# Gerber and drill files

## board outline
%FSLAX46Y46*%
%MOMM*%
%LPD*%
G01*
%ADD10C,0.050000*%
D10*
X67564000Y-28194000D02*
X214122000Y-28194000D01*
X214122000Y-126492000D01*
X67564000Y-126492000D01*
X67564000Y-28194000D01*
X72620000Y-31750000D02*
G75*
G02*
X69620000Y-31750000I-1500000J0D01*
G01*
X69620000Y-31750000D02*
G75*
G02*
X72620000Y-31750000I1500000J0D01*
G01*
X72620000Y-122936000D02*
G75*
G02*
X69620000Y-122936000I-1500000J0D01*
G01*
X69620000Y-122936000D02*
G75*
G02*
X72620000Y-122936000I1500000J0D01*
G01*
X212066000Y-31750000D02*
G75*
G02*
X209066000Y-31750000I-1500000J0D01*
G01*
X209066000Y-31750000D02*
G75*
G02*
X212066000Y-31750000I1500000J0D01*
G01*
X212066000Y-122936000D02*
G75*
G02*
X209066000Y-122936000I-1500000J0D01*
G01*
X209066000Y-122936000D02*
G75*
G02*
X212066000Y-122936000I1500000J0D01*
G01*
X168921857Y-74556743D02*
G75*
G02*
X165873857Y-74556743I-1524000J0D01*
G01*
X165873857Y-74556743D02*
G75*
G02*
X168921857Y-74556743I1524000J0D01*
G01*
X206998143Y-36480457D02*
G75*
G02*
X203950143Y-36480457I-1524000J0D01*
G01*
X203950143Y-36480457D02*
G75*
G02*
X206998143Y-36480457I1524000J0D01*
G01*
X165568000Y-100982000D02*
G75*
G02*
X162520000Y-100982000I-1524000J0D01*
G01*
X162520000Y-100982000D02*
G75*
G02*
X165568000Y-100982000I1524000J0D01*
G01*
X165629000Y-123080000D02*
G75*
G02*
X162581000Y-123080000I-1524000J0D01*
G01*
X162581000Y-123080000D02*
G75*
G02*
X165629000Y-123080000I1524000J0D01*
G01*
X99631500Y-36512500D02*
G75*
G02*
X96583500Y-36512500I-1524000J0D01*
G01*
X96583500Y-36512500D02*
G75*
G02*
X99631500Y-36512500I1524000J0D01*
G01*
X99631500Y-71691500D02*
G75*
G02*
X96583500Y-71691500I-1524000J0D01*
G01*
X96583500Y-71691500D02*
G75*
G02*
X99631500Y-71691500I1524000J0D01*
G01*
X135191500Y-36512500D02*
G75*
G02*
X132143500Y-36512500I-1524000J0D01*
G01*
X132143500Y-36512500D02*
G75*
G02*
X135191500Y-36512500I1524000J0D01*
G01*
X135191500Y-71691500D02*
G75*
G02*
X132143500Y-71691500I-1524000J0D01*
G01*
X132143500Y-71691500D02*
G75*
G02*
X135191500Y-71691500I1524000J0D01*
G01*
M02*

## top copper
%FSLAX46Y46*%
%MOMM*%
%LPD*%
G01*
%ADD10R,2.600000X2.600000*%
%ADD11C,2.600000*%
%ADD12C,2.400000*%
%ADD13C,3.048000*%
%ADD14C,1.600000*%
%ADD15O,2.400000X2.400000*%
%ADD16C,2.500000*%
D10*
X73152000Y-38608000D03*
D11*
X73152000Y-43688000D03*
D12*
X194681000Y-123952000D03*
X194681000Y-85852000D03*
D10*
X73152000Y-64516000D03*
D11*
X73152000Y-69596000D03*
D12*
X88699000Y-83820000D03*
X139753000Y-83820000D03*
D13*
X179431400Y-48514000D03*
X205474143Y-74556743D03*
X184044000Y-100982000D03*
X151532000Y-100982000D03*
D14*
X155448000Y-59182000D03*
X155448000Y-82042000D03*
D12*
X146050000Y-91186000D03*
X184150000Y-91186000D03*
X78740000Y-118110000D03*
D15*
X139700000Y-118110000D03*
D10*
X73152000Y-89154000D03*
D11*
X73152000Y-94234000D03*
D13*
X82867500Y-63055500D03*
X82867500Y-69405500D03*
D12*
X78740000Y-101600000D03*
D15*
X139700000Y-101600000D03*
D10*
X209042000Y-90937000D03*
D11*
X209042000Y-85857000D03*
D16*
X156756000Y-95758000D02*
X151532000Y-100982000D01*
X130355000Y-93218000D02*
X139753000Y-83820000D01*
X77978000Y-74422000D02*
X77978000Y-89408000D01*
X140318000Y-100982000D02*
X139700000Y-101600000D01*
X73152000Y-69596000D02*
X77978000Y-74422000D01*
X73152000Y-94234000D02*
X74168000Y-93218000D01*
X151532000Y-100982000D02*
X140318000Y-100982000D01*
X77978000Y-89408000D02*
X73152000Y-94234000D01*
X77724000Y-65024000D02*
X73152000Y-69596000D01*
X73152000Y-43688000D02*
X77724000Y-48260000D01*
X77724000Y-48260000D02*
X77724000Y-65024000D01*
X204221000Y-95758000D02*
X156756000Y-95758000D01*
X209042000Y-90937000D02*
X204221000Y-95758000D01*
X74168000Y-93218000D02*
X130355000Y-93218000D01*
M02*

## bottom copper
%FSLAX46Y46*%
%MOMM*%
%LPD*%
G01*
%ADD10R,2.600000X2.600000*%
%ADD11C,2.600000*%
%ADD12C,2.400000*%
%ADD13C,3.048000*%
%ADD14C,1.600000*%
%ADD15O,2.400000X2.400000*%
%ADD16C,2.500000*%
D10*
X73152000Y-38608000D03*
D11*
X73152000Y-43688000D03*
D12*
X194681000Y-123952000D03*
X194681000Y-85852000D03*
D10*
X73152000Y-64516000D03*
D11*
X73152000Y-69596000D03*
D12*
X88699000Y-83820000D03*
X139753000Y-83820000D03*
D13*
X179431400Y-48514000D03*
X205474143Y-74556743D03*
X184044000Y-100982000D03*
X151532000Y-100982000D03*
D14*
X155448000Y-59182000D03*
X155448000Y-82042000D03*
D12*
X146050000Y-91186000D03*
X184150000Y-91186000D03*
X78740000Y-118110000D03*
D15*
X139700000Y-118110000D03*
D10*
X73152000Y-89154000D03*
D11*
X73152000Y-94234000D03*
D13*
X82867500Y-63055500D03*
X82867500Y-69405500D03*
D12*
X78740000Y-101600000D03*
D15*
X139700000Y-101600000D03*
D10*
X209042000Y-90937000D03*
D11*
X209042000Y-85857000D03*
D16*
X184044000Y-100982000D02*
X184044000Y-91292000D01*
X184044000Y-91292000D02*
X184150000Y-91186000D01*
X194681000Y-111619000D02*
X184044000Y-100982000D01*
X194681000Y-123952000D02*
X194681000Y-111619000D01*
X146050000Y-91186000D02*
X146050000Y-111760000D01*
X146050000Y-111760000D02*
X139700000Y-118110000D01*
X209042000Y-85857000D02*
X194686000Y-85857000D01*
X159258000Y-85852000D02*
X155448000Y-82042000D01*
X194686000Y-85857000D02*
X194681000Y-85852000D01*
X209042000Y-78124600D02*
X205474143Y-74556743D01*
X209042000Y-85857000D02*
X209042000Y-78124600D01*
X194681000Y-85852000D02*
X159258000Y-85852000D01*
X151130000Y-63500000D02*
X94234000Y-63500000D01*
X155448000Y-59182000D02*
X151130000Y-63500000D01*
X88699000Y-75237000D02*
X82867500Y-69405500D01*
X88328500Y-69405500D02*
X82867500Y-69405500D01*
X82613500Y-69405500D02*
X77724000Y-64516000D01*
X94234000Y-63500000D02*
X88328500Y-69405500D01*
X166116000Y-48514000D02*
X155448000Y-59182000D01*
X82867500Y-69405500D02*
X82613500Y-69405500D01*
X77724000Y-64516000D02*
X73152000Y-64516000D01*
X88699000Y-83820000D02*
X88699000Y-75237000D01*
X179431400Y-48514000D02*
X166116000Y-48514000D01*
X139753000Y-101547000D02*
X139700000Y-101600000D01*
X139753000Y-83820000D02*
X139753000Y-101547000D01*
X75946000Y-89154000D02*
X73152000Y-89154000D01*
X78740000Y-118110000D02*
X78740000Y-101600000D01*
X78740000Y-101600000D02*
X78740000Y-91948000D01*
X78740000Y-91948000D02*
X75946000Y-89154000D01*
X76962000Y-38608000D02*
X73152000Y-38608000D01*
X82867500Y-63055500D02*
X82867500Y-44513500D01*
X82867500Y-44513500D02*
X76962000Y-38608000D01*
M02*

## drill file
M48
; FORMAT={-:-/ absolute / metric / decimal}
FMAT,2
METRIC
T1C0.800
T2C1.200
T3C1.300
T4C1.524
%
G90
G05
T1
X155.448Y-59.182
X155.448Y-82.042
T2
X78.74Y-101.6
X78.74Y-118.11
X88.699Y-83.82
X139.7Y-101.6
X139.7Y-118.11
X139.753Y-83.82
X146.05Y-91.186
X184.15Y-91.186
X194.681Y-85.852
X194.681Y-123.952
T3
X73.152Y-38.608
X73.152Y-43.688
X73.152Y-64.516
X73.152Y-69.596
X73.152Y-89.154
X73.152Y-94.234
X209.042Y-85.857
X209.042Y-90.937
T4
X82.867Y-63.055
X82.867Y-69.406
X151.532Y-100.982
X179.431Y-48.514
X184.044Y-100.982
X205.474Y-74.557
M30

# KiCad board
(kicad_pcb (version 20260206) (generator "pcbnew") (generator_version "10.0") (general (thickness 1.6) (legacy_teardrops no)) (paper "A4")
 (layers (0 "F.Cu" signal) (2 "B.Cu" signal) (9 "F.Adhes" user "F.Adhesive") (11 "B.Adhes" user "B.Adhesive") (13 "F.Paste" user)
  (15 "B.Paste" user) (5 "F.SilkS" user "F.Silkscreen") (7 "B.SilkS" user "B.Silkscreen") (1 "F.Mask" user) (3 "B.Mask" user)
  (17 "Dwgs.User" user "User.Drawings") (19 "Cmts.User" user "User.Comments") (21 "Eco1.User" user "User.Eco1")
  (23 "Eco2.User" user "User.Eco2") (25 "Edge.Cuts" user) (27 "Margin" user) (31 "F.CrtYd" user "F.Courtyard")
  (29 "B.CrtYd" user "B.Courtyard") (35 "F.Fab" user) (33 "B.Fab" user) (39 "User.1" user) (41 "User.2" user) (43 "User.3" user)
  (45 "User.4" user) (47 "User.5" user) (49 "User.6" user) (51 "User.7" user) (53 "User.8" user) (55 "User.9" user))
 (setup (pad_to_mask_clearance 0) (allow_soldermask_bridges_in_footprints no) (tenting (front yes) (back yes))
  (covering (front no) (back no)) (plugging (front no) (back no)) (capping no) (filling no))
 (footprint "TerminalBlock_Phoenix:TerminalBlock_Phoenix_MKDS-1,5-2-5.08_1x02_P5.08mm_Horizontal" (layer "F.Cu") (at 73.152 38.608 -90)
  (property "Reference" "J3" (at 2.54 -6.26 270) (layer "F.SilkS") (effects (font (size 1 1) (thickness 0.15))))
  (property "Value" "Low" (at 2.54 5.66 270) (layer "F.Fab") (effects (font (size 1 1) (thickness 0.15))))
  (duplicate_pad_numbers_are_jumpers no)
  (pad "1" thru_hole rect (at 0 0 270) (size 2.6 2.6) (drill 1.3) (layers "*.Cu" "*.Mask") (remove_unused_layers no) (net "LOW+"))
  (pad "2" thru_hole circle (at 5.08 0 270) (size 2.6 2.6) (drill 1.3) (layers "*.Cu" "*.Mask") (remove_unused_layers no) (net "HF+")))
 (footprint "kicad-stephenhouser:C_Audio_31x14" (layer "F.Cu") (at 194.681 123.952 90)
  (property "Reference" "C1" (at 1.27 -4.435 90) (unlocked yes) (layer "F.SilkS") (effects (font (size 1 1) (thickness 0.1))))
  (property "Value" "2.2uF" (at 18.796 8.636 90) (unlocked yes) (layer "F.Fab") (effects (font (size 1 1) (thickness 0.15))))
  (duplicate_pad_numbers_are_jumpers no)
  (pad "1" thru_hole circle (at 0 0 90) (size 2.4 2.4) (drill 1.2) (layers "*.Cu" "*.Mask") (remove_unused_layers no) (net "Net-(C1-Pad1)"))
  (pad "2" thru_hole circle (at 38.1 0 90) (size 2.4 2.4) (drill 1.2) (layers "*.Cu" "*.Mask") (remove_unused_layers no) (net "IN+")))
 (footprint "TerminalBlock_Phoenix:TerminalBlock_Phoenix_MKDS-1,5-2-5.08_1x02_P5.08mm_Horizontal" (layer "F.Cu") (at 73.152 64.516 -90)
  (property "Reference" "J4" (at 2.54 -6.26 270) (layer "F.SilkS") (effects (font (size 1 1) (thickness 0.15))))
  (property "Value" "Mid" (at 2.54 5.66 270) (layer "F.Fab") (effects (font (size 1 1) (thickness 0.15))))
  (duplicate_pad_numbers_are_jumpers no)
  (pad "1" thru_hole rect (at 0 0 270) (size 2.6 2.6) (drill 1.3) (layers "*.Cu" "*.Mask") (remove_unused_layers no) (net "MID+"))
  (pad "2" thru_hole circle (at 5.08 0 270) (size 2.6 2.6) (drill 1.3) (layers "*.Cu" "*.Mask") (remove_unused_layers no) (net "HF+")))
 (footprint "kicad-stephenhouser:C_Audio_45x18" (layer "F.Cu") (at 88.699 83.82)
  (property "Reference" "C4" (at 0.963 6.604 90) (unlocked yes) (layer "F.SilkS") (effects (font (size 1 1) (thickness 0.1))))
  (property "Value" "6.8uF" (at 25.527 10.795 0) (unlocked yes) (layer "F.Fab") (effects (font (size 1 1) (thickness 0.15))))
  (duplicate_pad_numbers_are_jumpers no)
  (pad "1" thru_hole circle (at 0 0) (size 2.4 2.4) (drill 1.2) (layers "*.Cu" "*.Mask") (remove_unused_layers no) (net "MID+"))
  (pad "2" thru_hole circle (at 51.054 0) (size 2.4 2.4) (drill 1.2) (layers "*.Cu" "*.Mask") (remove_unused_layers no) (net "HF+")))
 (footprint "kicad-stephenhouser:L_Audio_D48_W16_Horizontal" (layer "F.Cu") (at 186.436 55.5186 -45)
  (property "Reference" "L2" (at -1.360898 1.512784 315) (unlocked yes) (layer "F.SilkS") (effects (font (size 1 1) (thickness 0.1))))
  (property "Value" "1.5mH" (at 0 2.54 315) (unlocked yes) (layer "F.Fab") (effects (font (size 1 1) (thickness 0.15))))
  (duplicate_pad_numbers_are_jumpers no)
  (fp_circle (center 0 26.924) (end 1.524 26.924) (stroke (width 0.05) (type default)) (fill no) (layer "Edge.Cuts"))
  (fp_circle (center 0 -26.924) (end 1.524 -26.924) (stroke (width 0.05) (type default)) (fill no) (layer "Edge.Cuts"))
  (pad "1" thru_hole circle (at -9.906 0 315) (size 3.048 3.048) (drill 1.524) (layers "*.Cu" "*.Mask") (remove_unused_layers no)
   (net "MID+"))
  (pad "2" thru_hole circle (at 26.924 0 315) (size 3.048 3.048) (drill 1.524) (layers "*.Cu" "*.Mask") (remove_unused_layers no)
   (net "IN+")))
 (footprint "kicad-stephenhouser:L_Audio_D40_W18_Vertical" (layer "F.Cu") (at 184.044 100.982 180)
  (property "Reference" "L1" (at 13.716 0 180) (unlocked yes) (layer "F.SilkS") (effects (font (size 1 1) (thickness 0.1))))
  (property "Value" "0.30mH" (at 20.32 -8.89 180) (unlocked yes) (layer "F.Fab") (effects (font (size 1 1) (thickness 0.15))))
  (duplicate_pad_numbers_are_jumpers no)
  (fp_circle (center 20 0) (end 21.524 0) (stroke (width 0.05) (type default)) (fill no) (layer "Edge.Cuts"))
  (fp_circle (center 19.939 -22.098) (end 21.463 -22.098) (stroke (width 0.05) (type default)) (fill no) (layer "Edge.Cuts"))
  (pad "1" thru_hole circle (at 0 0 180) (size 3.048 3.048) (drill 1.524) (layers "*.Cu" "*.Mask") (remove_unused_layers no)
   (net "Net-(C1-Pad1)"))
  (pad "2" thru_hole circle (at 32.512 0 180) (size 3.048 3.048) (drill 1.524) (layers "*.Cu" "*.Mask") (remove_unused_layers no)
   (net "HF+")))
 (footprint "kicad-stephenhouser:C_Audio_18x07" (layer "F.Cu") (at 155.448 59.182 -90)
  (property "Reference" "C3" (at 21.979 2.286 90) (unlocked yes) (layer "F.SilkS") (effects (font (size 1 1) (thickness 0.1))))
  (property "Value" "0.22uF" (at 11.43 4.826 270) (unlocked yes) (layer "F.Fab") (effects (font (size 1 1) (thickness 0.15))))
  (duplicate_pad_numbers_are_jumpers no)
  (pad "1" thru_hole circle (at 0 0 270) (size 1.6 1.6) (drill 0.8) (layers "*.Cu" "*.Mask") (remove_unused_layers no) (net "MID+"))
  (pad "2" thru_hole circle (at 22.86 0 270) (size 1.6 1.6) (drill 0.8) (layers "*.Cu" "*.Mask") (remove_unused_layers no) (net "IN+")))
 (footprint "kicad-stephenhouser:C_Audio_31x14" (layer "F.Cu") (at 146.05 91.186)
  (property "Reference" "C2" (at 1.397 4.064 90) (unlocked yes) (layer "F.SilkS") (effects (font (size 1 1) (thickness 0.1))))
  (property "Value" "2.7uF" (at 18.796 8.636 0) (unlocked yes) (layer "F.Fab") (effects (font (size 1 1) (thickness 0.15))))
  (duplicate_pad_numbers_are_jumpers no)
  (pad "1" thru_hole circle (at 0 0) (size 2.4 2.4) (drill 1.2) (layers "*.Cu" "*.Mask") (remove_unused_layers no) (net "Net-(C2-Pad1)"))
  (pad "2" thru_hole circle (at 38.1 0) (size 2.4 2.4) (drill 1.2) (layers "*.Cu" "*.Mask") (remove_unused_layers no) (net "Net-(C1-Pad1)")))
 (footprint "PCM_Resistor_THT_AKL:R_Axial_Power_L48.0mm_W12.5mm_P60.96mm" (layer "F.Cu") (at 78.74 118.11)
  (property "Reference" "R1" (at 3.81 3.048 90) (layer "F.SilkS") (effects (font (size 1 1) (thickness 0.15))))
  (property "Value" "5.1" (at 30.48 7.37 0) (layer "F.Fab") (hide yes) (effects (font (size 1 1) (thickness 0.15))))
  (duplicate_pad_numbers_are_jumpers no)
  (pad "1" thru_hole circle (at 0 0) (size 2.4 2.4) (drill 1.2) (layers "*.Cu" "*.Mask") (remove_unused_layers no) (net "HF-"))
  (pad "2" thru_hole oval (at 60.96 0) (size 2.4 2.4) (drill 1.2) (layers "*.Cu" "*.Mask") (remove_unused_layers no) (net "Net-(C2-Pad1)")))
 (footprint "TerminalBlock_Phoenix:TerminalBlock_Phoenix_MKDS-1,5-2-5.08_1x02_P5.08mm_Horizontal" (layer "F.Cu") (at 73.152 89.154 -90)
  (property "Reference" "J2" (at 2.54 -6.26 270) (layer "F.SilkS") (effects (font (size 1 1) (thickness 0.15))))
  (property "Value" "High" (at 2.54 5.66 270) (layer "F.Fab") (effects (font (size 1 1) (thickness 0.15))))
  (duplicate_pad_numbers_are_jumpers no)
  (pad "1" thru_hole rect (at 0 0 270) (size 2.6 2.6) (drill 1.3) (layers "*.Cu" "*.Mask") (remove_unused_layers no) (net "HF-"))
  (pad "2" thru_hole circle (at 5.08 0 270) (size 2.6 2.6) (drill 1.3) (layers "*.Cu" "*.Mask") (remove_unused_layers no) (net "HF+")))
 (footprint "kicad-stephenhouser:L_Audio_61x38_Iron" (layer "F.Cu") (at 82.8675 69.4055)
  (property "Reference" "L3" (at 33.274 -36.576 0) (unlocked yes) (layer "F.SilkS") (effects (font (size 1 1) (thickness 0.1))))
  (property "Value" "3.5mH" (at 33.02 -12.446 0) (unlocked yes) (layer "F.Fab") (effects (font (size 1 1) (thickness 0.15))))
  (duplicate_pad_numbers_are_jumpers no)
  (fp_circle (center 15.24 -32.893) (end 16.764 -32.893) (stroke (width 0.05) (type default)) (fill no) (layer "Edge.Cuts"))
  (fp_circle (center 15.24 2.286) (end 16.764 2.286) (stroke (width 0.05) (type default)) (fill no) (layer "Edge.Cuts"))
  (fp_circle (center 50.8 -32.893) (end 52.324 -32.893) (stroke (width 0.05) (type default)) (fill no) (layer "Edge.Cuts"))
  (fp_circle (center 50.8 2.286) (end 52.324 2.286) (stroke (width 0.05) (type default)) (fill no) (layer "Edge.Cuts"))
  (pad "1" thru_hole circle (at 0 -6.35) (size 3.048 3.048) (drill 1.524) (layers "*.Cu" "*.Mask") (remove_unused_layers no) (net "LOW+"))
  (pad "2" thru_hole circle (at 0 0) (size 3.048 3.048) (drill 1.524) (layers "*.Cu" "*.Mask") (remove_unused_layers no) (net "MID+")))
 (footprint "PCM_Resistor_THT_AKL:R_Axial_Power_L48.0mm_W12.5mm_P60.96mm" (layer "F.Cu") (at 78.74 101.6)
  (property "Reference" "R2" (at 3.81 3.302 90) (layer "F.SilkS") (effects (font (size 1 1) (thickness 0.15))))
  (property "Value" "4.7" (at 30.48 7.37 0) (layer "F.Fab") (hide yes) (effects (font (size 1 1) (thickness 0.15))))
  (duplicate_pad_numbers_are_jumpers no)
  (pad "1" thru_hole circle (at 0 0) (size 2.4 2.4) (drill 1.2) (layers "*.Cu" "*.Mask") (remove_unused_layers no) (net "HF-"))
  (pad "2" thru_hole oval (at 60.96 0) (size 2.4 2.4) (drill 1.2) (layers "*.Cu" "*.Mask") (remove_unused_layers no) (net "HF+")))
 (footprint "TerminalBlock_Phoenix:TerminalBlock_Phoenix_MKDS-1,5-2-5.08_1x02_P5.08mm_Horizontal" (layer "F.Cu") (at 209.042 90.937 90)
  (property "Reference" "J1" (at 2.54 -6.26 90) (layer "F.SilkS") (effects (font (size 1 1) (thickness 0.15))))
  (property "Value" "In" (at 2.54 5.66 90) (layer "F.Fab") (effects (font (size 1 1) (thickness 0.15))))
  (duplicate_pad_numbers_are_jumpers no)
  (pad "1" thru_hole rect (at 0 0 90) (size 2.6 2.6) (drill 1.3) (layers "*.Cu" "*.Mask") (remove_unused_layers no) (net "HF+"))
  (pad "2" thru_hole circle (at 5.08 0 90) (size 2.6 2.6) (drill 1.3) (layers "*.Cu" "*.Mask") (remove_unused_layers no) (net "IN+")))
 (gr_rect (start 67.564 28.194) (end 214.122 126.492) (stroke (width 0.05) (type default)) (fill no) (layer "Edge.Cuts"))
 (gr_circle (center 71.12 31.75) (end 72.62 31.75) (stroke (width 0.05) (type default)) (fill no) (layer "Edge.Cuts"))
 (gr_circle (center 71.12 122.936) (end 72.62 122.936) (stroke (width 0.05) (type default)) (fill no) (layer "Edge.Cuts"))
 (gr_circle (center 210.566 31.75) (end 212.066 31.75) (stroke (width 0.05) (type default)) (fill no) (layer "Edge.Cuts"))
 (gr_circle (center 210.566 122.936) (end 212.066 122.936) (stroke (width 0.05) (type default)) (fill no) (layer "Edge.Cuts"))
 (segment (start 184.044 100.982) (end 184.044 91.292) (width 2.5) (layer "B.Cu") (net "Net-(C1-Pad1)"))
 (segment (start 184.044 91.292) (end 184.15 91.186) (width 2.5) (layer "B.Cu") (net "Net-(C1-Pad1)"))
 (segment (start 194.681 111.619) (end 184.044 100.982) (width 2.5) (layer "B.Cu") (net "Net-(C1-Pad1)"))
 (segment (start 194.681 123.952) (end 194.681 111.619) (width 2.5) (layer "B.Cu") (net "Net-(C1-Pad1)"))
 (segment (start 146.05 91.186) (end 146.05 111.76) (width 2.5) (layer "B.Cu") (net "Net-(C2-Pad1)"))
 (segment (start 146.05 111.76) (end 139.7 118.11) (width 2.5) (layer "B.Cu") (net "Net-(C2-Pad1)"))
 (segment (start 209.042 85.857) (end 194.686 85.857) (width 2.5) (layer "B.Cu") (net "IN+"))
 (segment (start 159.258 85.852) (end 155.448 82.042) (width 2.5) (layer "B.Cu") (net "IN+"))
 (segment (start 194.686 85.857) (end 194.681 85.852) (width 2.5) (layer "B.Cu") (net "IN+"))
 (segment (start 209.042 78.1246) (end 205.474143 74.556743) (width 2.5) (layer "B.Cu") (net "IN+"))
 (segment (start 209.042 85.857) (end 209.042 78.1246) (width 2.5) (layer "B.Cu") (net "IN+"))
 (segment (start 194.681 85.852) (end 159.258 85.852) (width 2.5) (layer "B.Cu") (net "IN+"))
 (segment (start 151.13 63.5) (end 94.234 63.5) (width 2.5) (layer "B.Cu") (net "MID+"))
 (segment (start 155.448 59.182) (end 151.13 63.5) (width 2.5) (layer "B.Cu") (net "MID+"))
 (segment (start 88.699 75.237) (end 82.8675 69.4055) (width 2.5) (layer "B.Cu") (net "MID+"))
 (segment (start 88.3285 69.4055) (end 82.8675 69.4055) (width 2.5) (layer "B.Cu") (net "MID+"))
 (segment (start 82.6135 69.4055) (end 77.724 64.516) (width 2.5) (layer "B.Cu") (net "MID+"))
 (segment (start 94.234 63.5) (end 88.3285 69.4055) (width 2.5) (layer "B.Cu") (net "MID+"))
 (segment (start 166.116 48.514) (end 155.448 59.182) (width 2.5) (layer "B.Cu") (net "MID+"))
 (segment (start 82.8675 69.4055) (end 82.6135 69.4055) (width 2.5) (layer "B.Cu") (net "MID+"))
 (segment (start 77.724 64.516) (end 73.152 64.516) (width 2.5) (layer "B.Cu") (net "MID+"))
 (segment (start 88.699 83.82) (end 88.699 75.237) (width 2.5) (layer "B.Cu") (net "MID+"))
 (segment (start 179.4314 48.514) (end 166.116 48.514) (width 2.5) (layer "B.Cu") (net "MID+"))
 (segment (start 156.756 95.758) (end 151.532 100.982) (width 2.5) (layer "F.Cu") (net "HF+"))
 (segment (start 130.355 93.218) (end 139.753 83.82) (width 2.5) (layer "F.Cu") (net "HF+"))
 (segment (start 77.978 74.422) (end 77.978 89.408) (width 2.5) (layer "F.Cu") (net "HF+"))
 (segment (start 140.318 100.982) (end 139.7 101.6) (width 2.5) (layer "F.Cu") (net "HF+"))
 (segment (start 73.152 69.596) (end 77.978 74.422) (width 2.5) (layer "F.Cu") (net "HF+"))
 (segment (start 73.152 94.234) (end 74.168 93.218) (width 2.5) (layer "F.Cu") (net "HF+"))
 (segment (start 151.532 100.982) (end 140.318 100.982) (width 2.5) (layer "F.Cu") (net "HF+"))
 (segment (start 77.978 89.408) (end 73.152 94.234) (width 2.5) (layer "F.Cu") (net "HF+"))
 (segment (start 77.724 65.024) (end 73.152 69.596) (width 2.5) (layer "F.Cu") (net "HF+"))
 (segment (start 73.152 43.688) (end 77.724 48.26) (width 2.5) (layer "F.Cu") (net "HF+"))
 (segment (start 77.724 48.26) (end 77.724 65.024) (width 2.5) (layer "F.Cu") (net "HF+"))
 (segment (start 204.221 95.758) (end 156.756 95.758) (width 2.5) (layer "F.Cu") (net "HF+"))
 (segment (start 209.042 90.937) (end 204.221 95.758) (width 2.5) (layer "F.Cu") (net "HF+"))
 (segment (start 74.168 93.218) (end 130.355 93.218) (width 2.5) (layer "F.Cu") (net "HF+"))
 (segment (start 139.753 101.547) (end 139.7 101.6) (width 2.5) (layer "B.Cu") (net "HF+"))
 (segment (start 139.753 83.82) (end 139.753 101.547) (width 2.5) (layer "B.Cu") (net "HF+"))
 (segment (start 75.946 89.154) (end 73.152 89.154) (width 2.5) (layer "B.Cu") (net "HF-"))
 (segment (start 78.74 118.11) (end 78.74 101.6) (width 2.5) (layer "B.Cu") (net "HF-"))
 (segment (start 78.74 101.6) (end 78.74 91.948) (width 2.5) (layer "B.Cu") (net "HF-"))
 (segment (start 78.74 91.948) (end 75.946 89.154) (width 2.5) (layer "B.Cu") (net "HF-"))
 (segment (start 76.962 38.608) (end 73.152 38.608) (width 2.5) (layer "B.Cu") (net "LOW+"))
 (segment (start 82.8675 63.0555) (end 82.8675 44.5135) (width 2.5) (layer "B.Cu") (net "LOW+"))
 (segment (start 82.8675 44.5135) (end 76.962 38.608) (width 2.5) (layer "B.Cu") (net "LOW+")))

